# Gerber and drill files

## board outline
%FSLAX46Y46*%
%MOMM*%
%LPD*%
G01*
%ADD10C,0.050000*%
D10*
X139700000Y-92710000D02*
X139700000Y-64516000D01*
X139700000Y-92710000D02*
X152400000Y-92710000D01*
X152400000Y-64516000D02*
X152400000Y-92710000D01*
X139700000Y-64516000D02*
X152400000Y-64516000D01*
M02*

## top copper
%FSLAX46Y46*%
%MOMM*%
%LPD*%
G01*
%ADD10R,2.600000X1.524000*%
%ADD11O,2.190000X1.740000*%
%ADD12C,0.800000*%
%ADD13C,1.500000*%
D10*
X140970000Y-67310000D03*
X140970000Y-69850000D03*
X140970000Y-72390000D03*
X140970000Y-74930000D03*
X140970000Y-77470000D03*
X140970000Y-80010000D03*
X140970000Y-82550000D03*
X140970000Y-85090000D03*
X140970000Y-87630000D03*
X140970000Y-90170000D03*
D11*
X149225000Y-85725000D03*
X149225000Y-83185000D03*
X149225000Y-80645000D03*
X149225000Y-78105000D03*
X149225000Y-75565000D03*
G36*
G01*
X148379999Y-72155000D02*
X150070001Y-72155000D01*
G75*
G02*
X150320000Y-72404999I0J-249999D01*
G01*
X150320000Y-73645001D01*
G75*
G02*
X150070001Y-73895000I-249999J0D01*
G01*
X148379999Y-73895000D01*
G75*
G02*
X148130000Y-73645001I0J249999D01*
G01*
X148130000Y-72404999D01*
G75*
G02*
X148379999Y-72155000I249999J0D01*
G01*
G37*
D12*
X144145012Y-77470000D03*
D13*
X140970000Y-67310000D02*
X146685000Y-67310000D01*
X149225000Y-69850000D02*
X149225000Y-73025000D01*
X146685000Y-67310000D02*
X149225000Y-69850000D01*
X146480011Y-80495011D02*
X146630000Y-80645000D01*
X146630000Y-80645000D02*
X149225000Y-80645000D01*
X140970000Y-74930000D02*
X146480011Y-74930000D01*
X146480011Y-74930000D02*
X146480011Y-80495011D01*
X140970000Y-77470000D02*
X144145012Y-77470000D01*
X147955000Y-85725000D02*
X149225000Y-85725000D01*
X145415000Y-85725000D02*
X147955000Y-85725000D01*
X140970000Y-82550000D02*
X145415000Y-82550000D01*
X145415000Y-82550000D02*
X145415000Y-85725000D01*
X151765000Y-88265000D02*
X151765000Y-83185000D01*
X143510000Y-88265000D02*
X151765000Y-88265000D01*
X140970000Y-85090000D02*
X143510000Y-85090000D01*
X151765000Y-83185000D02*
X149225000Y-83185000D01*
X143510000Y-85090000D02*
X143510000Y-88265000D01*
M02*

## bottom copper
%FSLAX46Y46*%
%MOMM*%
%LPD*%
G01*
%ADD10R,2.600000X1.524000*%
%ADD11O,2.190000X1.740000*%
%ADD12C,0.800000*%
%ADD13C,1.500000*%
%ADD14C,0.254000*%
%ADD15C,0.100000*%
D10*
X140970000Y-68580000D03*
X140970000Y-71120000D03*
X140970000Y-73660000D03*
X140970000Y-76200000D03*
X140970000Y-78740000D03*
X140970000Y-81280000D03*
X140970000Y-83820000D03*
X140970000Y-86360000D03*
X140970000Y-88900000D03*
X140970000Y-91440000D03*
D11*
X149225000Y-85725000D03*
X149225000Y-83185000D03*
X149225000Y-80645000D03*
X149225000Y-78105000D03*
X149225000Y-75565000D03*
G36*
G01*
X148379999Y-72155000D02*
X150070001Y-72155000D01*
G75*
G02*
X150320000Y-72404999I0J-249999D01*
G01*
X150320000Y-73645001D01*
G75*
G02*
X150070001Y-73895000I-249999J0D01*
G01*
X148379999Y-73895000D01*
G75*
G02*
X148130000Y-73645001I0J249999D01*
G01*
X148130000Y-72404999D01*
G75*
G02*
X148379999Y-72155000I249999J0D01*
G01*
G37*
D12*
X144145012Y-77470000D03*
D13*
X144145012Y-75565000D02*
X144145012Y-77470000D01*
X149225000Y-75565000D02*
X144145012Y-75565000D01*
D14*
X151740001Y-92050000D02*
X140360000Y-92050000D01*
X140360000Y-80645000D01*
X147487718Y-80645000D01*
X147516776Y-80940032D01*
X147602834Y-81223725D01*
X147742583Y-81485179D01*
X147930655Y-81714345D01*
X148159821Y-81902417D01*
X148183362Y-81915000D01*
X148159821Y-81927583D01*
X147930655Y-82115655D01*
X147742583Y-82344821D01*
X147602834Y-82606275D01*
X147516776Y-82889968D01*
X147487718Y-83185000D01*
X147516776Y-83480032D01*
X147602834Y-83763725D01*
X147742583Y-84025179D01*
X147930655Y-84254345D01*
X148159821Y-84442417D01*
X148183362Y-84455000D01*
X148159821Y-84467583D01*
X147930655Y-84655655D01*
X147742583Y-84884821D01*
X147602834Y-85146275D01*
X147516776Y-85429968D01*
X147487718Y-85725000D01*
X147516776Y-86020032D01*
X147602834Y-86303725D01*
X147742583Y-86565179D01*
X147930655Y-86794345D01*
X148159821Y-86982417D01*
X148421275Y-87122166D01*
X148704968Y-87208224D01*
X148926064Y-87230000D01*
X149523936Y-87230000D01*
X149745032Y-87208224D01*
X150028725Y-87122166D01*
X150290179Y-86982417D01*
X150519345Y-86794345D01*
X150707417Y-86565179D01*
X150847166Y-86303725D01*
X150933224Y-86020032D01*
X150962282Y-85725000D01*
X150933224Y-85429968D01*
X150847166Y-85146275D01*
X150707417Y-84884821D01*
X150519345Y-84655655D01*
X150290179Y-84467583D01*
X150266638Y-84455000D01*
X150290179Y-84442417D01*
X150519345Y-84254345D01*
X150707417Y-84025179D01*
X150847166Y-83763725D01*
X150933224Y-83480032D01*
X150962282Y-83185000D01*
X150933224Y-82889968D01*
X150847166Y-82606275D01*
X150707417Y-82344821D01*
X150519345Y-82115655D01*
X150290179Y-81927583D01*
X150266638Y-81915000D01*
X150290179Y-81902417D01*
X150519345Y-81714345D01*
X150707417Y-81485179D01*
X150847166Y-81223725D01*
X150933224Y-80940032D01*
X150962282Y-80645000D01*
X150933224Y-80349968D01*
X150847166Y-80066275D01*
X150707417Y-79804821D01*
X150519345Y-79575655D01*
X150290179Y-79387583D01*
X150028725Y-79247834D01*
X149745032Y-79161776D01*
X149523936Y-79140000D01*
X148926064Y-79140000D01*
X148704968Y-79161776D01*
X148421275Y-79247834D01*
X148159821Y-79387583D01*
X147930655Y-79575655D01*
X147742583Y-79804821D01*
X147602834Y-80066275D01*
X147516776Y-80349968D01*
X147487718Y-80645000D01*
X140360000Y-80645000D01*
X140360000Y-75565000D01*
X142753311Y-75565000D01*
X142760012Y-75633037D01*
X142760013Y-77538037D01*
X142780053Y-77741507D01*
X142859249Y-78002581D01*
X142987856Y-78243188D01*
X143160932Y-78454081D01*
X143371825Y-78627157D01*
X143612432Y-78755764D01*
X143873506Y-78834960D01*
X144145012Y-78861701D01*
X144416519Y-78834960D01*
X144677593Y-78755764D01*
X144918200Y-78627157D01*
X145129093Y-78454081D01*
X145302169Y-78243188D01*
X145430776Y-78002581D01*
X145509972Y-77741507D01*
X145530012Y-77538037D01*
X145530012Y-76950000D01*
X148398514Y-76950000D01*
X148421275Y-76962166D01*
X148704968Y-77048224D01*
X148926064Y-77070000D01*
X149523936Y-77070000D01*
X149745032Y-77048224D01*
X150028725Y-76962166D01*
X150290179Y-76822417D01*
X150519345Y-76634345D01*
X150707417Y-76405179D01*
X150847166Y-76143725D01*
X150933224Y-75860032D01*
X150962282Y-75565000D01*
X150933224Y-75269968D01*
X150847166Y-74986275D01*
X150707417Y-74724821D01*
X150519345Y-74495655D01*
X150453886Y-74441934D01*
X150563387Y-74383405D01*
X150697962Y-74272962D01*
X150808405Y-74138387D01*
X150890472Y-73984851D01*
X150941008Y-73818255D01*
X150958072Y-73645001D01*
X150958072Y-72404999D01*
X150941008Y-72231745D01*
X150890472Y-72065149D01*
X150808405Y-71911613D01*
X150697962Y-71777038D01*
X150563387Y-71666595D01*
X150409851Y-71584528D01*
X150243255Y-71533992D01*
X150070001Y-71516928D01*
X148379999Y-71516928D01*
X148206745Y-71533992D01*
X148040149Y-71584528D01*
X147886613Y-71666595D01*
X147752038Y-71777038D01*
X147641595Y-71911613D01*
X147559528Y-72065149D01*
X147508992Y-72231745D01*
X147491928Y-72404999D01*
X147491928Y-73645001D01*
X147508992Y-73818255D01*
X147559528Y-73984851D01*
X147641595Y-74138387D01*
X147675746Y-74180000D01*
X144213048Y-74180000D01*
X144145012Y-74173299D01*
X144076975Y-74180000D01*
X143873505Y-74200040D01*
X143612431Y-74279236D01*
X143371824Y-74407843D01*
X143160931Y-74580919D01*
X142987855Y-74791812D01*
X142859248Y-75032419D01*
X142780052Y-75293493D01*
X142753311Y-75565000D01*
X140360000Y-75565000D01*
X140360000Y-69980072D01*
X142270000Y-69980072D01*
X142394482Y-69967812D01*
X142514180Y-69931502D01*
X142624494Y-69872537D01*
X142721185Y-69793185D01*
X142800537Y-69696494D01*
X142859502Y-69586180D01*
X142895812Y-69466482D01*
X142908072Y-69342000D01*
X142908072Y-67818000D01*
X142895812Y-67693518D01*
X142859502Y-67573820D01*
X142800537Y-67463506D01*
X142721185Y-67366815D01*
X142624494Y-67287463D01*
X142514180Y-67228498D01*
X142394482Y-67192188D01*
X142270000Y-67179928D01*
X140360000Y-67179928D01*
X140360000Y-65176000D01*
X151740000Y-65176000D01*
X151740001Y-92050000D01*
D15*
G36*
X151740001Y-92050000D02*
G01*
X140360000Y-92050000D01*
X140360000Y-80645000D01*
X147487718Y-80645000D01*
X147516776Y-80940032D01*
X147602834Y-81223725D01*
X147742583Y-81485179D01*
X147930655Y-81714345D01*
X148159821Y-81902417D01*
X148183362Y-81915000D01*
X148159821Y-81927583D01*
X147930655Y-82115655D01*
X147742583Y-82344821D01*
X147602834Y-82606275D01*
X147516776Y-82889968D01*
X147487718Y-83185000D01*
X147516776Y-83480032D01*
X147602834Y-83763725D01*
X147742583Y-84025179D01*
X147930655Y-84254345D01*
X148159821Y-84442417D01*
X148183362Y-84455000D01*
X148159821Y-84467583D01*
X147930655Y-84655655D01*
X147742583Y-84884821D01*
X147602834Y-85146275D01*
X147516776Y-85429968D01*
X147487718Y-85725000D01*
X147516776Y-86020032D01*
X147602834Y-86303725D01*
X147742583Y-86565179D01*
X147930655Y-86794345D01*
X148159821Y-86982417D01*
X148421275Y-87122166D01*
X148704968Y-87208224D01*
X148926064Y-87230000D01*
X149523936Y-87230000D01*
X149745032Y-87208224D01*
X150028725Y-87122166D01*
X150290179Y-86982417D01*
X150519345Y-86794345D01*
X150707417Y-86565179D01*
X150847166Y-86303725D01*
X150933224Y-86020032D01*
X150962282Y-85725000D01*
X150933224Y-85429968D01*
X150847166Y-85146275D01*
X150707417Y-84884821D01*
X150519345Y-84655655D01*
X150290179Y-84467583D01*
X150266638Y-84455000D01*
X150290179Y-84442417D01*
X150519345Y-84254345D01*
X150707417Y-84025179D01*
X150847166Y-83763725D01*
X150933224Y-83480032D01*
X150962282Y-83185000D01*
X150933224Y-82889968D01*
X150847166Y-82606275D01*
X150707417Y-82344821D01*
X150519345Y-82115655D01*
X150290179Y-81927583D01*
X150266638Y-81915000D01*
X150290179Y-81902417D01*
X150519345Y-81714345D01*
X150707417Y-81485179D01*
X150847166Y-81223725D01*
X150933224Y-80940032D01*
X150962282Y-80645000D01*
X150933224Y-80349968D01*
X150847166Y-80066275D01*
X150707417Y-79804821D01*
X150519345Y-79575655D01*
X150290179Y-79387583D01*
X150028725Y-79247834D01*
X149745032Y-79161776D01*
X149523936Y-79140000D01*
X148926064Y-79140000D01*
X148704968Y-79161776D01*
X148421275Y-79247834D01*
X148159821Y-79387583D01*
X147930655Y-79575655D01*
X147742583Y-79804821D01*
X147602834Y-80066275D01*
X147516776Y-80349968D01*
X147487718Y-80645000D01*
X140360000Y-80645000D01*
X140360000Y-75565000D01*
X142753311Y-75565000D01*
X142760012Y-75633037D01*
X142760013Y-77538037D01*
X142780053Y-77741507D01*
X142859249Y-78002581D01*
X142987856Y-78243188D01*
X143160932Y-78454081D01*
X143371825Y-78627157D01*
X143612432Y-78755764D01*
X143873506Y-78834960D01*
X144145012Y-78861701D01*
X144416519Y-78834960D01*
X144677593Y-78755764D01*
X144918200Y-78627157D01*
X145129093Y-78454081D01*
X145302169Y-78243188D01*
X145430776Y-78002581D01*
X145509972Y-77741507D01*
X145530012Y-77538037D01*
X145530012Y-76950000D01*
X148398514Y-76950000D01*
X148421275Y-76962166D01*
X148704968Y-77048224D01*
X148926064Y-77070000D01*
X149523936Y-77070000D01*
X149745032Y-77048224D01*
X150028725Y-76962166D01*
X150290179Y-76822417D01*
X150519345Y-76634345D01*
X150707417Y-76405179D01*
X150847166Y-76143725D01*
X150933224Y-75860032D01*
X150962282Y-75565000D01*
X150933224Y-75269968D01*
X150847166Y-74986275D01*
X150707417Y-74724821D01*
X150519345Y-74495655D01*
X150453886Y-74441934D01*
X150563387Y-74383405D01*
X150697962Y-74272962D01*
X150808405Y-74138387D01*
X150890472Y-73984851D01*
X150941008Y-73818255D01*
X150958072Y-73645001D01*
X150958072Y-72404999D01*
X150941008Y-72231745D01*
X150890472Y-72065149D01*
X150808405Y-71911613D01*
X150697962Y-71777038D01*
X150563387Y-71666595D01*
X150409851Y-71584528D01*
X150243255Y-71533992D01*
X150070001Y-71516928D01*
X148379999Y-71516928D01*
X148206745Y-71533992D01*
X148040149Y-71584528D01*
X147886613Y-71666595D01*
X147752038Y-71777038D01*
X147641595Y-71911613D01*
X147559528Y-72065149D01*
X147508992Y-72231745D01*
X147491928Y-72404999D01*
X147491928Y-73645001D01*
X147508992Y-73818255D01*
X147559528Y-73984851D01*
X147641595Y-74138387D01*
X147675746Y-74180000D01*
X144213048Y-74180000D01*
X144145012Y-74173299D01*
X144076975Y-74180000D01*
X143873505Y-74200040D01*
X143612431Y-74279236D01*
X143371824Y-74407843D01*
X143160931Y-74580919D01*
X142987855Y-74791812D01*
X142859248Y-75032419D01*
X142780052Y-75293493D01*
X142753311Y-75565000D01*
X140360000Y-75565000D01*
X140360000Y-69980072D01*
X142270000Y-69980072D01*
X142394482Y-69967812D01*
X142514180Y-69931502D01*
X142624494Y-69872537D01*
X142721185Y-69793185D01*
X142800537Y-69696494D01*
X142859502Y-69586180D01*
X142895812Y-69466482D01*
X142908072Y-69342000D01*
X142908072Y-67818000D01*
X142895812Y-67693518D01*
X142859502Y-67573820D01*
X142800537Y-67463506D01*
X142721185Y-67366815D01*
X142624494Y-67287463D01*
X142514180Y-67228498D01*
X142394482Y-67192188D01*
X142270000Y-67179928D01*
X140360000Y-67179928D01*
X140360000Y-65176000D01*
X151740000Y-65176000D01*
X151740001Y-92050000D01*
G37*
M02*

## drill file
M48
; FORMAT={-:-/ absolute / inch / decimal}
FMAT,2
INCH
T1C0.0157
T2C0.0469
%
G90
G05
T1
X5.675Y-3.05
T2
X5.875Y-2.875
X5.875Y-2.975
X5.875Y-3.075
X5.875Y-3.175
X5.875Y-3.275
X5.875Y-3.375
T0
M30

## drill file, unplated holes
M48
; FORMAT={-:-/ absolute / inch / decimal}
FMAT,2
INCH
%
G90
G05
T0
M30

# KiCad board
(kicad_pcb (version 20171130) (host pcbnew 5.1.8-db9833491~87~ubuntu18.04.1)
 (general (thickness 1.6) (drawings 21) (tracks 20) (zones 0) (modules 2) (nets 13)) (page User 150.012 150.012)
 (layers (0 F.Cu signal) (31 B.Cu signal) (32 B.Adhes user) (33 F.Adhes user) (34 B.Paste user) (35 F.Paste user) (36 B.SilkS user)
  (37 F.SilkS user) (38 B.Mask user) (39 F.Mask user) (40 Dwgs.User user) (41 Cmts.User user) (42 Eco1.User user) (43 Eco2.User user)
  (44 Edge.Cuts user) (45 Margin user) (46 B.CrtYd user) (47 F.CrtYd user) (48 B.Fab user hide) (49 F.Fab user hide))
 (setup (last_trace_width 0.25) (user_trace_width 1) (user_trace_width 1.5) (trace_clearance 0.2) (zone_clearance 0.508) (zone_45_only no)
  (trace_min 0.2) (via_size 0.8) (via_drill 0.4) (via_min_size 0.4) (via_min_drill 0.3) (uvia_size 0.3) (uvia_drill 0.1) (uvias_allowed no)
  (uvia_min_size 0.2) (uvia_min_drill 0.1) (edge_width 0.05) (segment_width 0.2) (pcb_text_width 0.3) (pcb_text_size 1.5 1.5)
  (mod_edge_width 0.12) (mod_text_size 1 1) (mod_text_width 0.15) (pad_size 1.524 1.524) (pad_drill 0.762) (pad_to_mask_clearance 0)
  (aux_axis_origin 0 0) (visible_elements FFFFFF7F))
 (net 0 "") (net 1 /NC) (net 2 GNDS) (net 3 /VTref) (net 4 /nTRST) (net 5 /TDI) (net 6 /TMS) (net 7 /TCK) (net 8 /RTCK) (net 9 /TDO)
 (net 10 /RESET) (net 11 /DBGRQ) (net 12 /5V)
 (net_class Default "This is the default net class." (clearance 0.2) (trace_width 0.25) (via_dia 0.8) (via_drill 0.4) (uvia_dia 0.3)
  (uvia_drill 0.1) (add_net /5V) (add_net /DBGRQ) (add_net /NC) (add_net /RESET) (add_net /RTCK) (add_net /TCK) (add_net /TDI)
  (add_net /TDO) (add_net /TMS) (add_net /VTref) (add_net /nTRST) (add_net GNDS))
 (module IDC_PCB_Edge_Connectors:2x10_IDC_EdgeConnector (layer F.Cu) (at 71.374 64.389 90)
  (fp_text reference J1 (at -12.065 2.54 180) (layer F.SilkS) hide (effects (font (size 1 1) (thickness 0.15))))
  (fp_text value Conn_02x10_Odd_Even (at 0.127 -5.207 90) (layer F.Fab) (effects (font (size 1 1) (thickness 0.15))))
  (pad 2 smd rect (at 10.795 0 90) (size 1.524 2.6) (layers B.Cu B.Paste B.Mask) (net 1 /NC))
  (pad 4 smd rect (at 8.255 0 90) (size 1.524 2.6) (layers B.Cu B.Paste B.Mask) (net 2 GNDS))
  (pad 6 smd rect (at 5.715 0 90) (size 1.524 2.6) (layers B.Cu B.Paste B.Mask) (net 2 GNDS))
  (pad 8 smd rect (at 3.175 0 90) (size 1.524 2.6) (layers B.Cu B.Paste B.Mask) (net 2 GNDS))
  (pad 10 smd rect (at 0.635 0 90) (size 1.524 2.6) (layers B.Cu B.Paste B.Mask) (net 2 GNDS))
  (pad 12 smd rect (at -1.905 0 90) (size 1.524 2.6) (layers B.Cu B.Paste B.Mask) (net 2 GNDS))
  (pad 14 smd rect (at -4.445 0 90) (size 1.524 2.6) (layers B.Cu B.Paste B.Mask) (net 2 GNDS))
  (pad 16 smd rect (at -6.985 0 90) (size 1.524 2.6) (layers B.Cu B.Paste B.Mask) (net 2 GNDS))
  (pad 18 smd rect (at -9.525 0 90) (size 1.524 2.6) (layers B.Cu B.Paste B.Mask) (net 2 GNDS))
  (pad 20 smd rect (at -12.065 0 90) (size 1.524 2.6) (layers B.Cu B.Paste B.Mask) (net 2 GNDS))
  (pad 1 smd rect (at 12.065 0 90) (size 1.524 2.6) (layers F.Cu F.Paste F.Mask) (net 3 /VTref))
  (pad 3 smd rect (at 9.525 0 90) (size 1.524 2.6) (layers F.Cu F.Paste F.Mask) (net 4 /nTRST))
  (pad 5 smd rect (at 6.985 0 90) (size 1.524 2.6) (layers F.Cu F.Paste F.Mask) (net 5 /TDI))
  (pad 7 smd rect (at 4.445 0 90) (size 1.524 2.6) (layers F.Cu F.Paste F.Mask) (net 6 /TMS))
  (pad 9 smd rect (at 1.905 0 90) (size 1.524 2.6) (layers F.Cu F.Paste F.Mask) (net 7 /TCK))
  (pad 11 smd rect (at -0.635 0 90) (size 1.524 2.6) (layers F.Cu F.Paste F.Mask) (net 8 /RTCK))
  (pad 13 smd rect (at -3.175 0 90) (size 1.524 2.6) (layers F.Cu F.Paste F.Mask) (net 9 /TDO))
  (pad 15 smd rect (at -5.715 0 90) (size 1.524 2.6) (layers F.Cu F.Paste F.Mask) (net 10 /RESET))
  (pad 17 smd rect (at -8.255 0 90) (size 1.524 2.6) (layers F.Cu F.Paste F.Mask) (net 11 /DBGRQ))
  (pad 19 smd rect (at -10.795 0 90) (size 1.524 2.6) (layers F.Cu F.Paste F.Mask) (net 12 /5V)))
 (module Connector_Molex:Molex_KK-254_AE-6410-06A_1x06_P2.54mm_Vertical (layer F.Cu) (at 79.629 58.039 270)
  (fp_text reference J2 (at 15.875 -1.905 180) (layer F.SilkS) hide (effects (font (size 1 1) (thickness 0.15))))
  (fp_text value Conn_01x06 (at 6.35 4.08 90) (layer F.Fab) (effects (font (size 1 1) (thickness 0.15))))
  (pad 6 thru_hole oval (at 12.7 0 270) (size 1.74 2.19) (drill 1.19) (layers *.Cu *.Mask) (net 9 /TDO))
  (pad 5 thru_hole oval (at 10.16 0 270) (size 1.74 2.19) (drill 1.19) (layers *.Cu *.Mask) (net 10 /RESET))
  (pad 4 thru_hole oval (at 7.62 0 270) (size 1.74 2.19) (drill 1.19) (layers *.Cu *.Mask) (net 6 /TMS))
  (pad 3 thru_hole oval (at 5.08 0 270) (size 1.74 2.19) (drill 1.19) (layers *.Cu *.Mask) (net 2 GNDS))
  (pad 2 thru_hole oval (at 2.54 0 270) (size 1.74 2.19) (drill 1.19) (layers *.Cu *.Mask) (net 7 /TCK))
  (pad 1 thru_hole roundrect (at 0 0 270) (size 1.74 2.19) (drill 1.19) (layers *.Cu *.Mask) (roundrect_rratio 0.1436775862068966)
   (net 3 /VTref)))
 (gr_line (start 70.104 77.724) (end 70.104 49.53) (layer Edge.Cuts) (width 0.05))
 (gr_line (start 70.104 77.724) (end 82.804 77.724) (layer Edge.Cuts) (width 0.05))
 (gr_line (start 82.804 49.53) (end 82.804 77.724) (layer Edge.Cuts) (width 0.05))
 (gr_line (start 70.104 49.53) (end 82.804 49.53) (layer Edge.Cuts) (width 0.05))
 (segment (start 71.374 52.324) (end 77.089 52.324) (width 1.5) (layer F.Cu) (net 3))
 (segment (start 79.629 54.864) (end 79.629 58.039) (width 1.5) (layer F.Cu) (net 3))
 (segment (start 77.089 52.324) (end 79.629 54.864) (width 1.5) (layer F.Cu) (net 3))
 (segment (start 76.884011 65.509011) (end 77.034 65.659) (width 1.5) (layer F.Cu) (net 6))
 (segment (start 77.034 65.659) (end 79.629 65.659) (width 1.5) (layer F.Cu) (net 6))
 (segment (start 71.374 59.944) (end 76.884011 59.944) (width 1.5) (layer F.Cu) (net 6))
 (segment (start 76.884011 59.944) (end 76.884011 65.509011) (width 1.5) (layer F.Cu) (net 6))
 (via (at 74.549012 62.484) (size 0.8) (drill 0.4) (layers F.Cu B.Cu) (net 7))
 (segment (start 71.374 62.484) (end 74.549012 62.484) (width 1.5) (layer F.Cu) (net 7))
 (segment (start 74.549012 60.579) (end 74.549012 62.484) (width 1.5) (layer B.Cu) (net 7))
 (segment (start 79.629 60.579) (end 74.549012 60.579) (width 1.5) (layer B.Cu) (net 7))
 (segment (start 78.359 70.739) (end 79.629 70.739) (width 1.5) (layer F.Cu) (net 9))
 (segment (start 75.819 70.739) (end 78.359 70.739) (width 1.5) (layer F.Cu) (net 9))
 (segment (start 71.374 67.564) (end 75.819 67.564) (width 1.5) (layer F.Cu) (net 9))
 (segment (start 75.819 67.564) (end 75.819 70.739) (width 1.5) (layer F.Cu) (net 9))
 (segment (start 82.169 73.279) (end 82.169 68.199) (width 1.5) (layer F.Cu) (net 10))
 (segment (start 73.914 73.279) (end 82.169 73.279) (width 1.5) (layer F.Cu) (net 10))
 (segment (start 71.374 70.104) (end 73.914 70.104) (width 1.5) (layer F.Cu) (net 10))
 (segment (start 82.169 68.199) (end 79.629 68.199) (width 1.5) (layer F.Cu) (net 10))
 (segment (start 73.914 70.104) (end 73.914 73.279) (width 1.5) (layer F.Cu) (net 10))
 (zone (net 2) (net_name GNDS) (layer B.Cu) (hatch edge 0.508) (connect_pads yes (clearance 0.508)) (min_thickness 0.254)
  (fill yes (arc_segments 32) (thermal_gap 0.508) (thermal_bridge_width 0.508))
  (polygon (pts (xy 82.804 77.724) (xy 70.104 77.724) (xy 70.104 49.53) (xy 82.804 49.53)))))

